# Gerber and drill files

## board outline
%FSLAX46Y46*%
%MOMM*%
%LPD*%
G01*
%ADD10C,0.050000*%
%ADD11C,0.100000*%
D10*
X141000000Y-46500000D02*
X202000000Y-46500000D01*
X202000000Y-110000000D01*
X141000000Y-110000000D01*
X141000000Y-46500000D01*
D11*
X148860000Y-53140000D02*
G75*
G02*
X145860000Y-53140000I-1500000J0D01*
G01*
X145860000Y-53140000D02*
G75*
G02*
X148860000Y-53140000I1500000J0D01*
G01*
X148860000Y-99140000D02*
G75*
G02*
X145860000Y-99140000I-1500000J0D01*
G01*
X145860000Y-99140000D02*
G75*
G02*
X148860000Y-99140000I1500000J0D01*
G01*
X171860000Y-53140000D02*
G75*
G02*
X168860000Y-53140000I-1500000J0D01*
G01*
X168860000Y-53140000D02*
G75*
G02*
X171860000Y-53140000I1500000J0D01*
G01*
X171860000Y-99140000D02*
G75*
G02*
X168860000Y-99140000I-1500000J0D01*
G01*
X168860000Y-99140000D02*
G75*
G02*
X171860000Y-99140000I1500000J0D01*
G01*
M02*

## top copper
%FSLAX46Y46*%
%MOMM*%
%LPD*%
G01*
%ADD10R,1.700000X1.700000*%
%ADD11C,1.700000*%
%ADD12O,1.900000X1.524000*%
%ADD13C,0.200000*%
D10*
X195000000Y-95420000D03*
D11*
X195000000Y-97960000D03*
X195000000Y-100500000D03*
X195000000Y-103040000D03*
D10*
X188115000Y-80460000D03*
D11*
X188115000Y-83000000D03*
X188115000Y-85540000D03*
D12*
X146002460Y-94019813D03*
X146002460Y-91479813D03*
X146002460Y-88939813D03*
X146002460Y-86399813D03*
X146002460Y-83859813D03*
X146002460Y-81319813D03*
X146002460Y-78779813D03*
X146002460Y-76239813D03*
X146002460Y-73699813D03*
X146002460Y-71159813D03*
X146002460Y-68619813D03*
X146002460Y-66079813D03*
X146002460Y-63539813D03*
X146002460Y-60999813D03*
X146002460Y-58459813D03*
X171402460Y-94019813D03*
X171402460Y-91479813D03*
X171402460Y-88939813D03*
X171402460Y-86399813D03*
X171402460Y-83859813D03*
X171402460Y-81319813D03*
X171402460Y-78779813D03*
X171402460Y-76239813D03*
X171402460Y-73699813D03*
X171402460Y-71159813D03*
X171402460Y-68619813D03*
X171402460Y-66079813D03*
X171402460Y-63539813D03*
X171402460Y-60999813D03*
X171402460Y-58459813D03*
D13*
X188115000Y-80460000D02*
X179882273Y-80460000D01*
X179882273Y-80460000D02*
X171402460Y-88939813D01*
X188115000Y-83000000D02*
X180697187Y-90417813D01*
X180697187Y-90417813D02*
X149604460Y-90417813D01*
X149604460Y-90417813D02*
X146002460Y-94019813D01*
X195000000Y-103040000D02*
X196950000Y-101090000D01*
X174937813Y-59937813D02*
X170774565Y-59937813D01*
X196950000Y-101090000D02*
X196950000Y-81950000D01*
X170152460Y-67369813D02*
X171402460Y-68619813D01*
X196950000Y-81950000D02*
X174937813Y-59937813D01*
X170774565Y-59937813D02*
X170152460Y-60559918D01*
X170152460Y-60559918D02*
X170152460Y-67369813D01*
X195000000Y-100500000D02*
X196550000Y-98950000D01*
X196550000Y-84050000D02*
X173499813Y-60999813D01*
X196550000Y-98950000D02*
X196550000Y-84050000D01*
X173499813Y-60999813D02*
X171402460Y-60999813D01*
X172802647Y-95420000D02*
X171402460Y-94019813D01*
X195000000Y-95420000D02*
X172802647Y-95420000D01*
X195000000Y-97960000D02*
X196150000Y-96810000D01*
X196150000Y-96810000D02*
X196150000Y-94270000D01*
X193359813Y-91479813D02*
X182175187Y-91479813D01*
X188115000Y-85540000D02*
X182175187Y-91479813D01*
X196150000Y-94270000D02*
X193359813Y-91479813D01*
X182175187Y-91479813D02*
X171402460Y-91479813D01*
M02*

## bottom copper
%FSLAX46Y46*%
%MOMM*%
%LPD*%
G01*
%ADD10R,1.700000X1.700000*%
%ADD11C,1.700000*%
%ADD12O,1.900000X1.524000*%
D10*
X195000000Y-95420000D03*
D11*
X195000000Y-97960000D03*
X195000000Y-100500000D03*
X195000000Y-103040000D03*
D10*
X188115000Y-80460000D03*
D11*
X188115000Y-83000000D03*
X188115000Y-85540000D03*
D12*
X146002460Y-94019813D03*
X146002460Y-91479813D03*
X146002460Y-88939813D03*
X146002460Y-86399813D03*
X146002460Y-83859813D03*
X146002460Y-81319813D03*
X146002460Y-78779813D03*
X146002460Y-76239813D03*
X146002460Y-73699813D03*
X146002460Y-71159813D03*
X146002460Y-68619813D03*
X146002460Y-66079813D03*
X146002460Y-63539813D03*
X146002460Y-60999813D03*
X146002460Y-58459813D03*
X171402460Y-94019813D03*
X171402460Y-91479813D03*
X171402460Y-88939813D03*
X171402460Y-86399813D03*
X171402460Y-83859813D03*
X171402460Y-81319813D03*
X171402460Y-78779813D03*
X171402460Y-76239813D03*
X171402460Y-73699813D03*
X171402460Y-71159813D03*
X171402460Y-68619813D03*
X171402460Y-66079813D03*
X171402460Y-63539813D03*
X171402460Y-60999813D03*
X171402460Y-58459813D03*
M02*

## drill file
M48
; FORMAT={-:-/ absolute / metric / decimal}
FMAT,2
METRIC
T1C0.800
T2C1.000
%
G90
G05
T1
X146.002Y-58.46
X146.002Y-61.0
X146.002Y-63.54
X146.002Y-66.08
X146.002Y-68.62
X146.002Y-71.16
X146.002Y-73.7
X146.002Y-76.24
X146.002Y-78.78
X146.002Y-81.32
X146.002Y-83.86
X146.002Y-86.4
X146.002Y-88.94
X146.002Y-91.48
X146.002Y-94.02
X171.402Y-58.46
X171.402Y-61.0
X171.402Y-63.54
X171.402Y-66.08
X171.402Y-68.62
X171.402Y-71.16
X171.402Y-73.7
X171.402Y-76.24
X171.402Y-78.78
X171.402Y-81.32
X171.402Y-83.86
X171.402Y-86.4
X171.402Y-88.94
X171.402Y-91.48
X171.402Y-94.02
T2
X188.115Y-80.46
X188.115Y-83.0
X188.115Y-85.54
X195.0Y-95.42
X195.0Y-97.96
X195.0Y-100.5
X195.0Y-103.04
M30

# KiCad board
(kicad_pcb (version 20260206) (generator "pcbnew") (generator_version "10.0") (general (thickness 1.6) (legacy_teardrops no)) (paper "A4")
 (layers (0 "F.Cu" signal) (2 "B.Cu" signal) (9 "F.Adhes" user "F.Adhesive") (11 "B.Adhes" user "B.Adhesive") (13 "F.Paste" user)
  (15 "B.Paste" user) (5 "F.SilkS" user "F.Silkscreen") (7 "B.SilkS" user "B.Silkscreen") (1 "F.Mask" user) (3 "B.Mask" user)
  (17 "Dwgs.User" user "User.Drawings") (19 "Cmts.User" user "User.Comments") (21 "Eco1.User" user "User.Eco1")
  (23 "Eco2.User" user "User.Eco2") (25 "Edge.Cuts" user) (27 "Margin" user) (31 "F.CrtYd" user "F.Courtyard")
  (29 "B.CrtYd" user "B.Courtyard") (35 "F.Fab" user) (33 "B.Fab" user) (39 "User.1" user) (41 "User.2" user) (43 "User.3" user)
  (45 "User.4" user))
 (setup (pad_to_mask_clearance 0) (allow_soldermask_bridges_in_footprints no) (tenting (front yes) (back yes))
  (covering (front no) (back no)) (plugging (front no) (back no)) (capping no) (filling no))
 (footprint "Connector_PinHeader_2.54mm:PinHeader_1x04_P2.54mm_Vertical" (layer "F.Cu") (at 195 95.42)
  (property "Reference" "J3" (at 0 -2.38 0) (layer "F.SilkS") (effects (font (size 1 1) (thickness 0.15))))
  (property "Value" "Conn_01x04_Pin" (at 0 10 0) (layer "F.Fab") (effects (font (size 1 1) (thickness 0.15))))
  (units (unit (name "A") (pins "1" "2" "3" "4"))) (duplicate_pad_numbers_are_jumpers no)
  (pad "1" thru_hole rect (at 0 0) (size 1.7 1.7) (drill 1) (layers "*.Cu" "*.Mask") (remove_unused_layers no) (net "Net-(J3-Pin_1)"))
  (pad "2" thru_hole circle (at 0 2.54) (size 1.7 1.7) (drill 1) (layers "*.Cu" "*.Mask") (remove_unused_layers no) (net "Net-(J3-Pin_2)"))
  (pad "3" thru_hole circle (at 0 5.08) (size 1.7 1.7) (drill 1) (layers "*.Cu" "*.Mask") (remove_unused_layers no) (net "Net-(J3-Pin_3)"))
  (pad "4" thru_hole circle (at 0 7.62) (size 1.7 1.7) (drill 1) (layers "*.Cu" "*.Mask") (remove_unused_layers no) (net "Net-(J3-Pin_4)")))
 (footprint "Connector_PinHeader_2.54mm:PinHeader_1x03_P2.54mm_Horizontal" (layer "F.Cu") (at 188.115 80.46)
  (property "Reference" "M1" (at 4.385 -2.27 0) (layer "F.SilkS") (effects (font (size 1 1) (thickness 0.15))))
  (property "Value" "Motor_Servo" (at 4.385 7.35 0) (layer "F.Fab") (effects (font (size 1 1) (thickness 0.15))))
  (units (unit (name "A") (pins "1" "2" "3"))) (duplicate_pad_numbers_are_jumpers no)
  (pad "1" thru_hole rect (at 0 0) (size 1.7 1.7) (drill 1) (layers "*.Cu" "*.Mask") (remove_unused_layers no) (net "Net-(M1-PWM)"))
  (pad "2" thru_hole circle (at 0 2.54) (size 1.7 1.7) (drill 1) (layers "*.Cu" "*.Mask") (remove_unused_layers no) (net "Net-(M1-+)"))
  (pad "3" thru_hole circle (at 0 5.08) (size 1.7 1.7) (drill 1) (layers "*.Cu" "*.Mask") (remove_unused_layers no) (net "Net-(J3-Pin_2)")))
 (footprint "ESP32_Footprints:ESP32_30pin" (layer "F.Cu") (at 157.93 77)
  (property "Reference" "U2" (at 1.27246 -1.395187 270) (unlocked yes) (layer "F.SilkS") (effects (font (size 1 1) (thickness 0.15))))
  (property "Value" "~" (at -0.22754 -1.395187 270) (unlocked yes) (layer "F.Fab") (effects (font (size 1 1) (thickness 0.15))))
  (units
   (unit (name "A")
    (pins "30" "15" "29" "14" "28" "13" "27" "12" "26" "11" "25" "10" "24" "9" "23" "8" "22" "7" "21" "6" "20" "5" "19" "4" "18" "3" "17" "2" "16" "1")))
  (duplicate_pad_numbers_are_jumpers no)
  (fp_circle (center -10.57 -23.86) (end -10.57 -22.36) (stroke (width 0.1) (type default)) (fill no) (layer "Edge.Cuts"))
  (fp_circle (center -10.57 22.14) (end -10.57 23.64) (stroke (width 0.1) (type default)) (fill no) (layer "Edge.Cuts"))
  (fp_circle (center 12.43 -23.86) (end 12.43 -22.36) (stroke (width 0.1) (type default)) (fill no) (layer "Edge.Cuts"))
  (fp_circle (center 12.43 22.14) (end 12.43 23.64) (stroke (width 0.1) (type default)) (fill no) (layer "Edge.Cuts"))
  (pad "1" thru_hole oval (at -11.92754 17.019813 270) (size 1.524 1.9) (drill 0.8) (layers "*.Cu" "*.Mask") (remove_unused_layers no)
   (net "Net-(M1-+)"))
  (pad "2" thru_hole oval (at -11.92754 14.479813 270) (size 1.524 1.9) (drill 0.8) (layers "*.Cu" "*.Mask") (remove_unused_layers no)
   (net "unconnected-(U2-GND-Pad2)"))
  (pad "3" thru_hole oval (at -11.92754 11.939813 270) (size 1.524 1.9) (drill 0.8) (layers "*.Cu" "*.Mask") (remove_unused_layers no)
   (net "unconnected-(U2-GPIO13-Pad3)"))
  (pad "4" thru_hole oval (at -11.92754 9.399813 270) (size 1.524 1.9) (drill 0.8) (layers "*.Cu" "*.Mask") (remove_unused_layers no)
   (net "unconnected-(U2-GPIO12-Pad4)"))
  (pad "5" thru_hole oval (at -11.92754 6.859813 270) (size 1.524 1.9) (drill 0.8) (layers "*.Cu" "*.Mask") (remove_unused_layers no)
   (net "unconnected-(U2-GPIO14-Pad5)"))
  (pad "6" thru_hole oval (at -11.92754 4.319813 270) (size 1.524 1.9) (drill 0.8) (layers "*.Cu" "*.Mask") (remove_unused_layers no)
   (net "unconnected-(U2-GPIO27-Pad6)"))
  (pad "7" thru_hole oval (at -11.92754 1.779813 270) (size 1.524 1.9) (drill 0.8) (layers "*.Cu" "*.Mask") (remove_unused_layers no)
   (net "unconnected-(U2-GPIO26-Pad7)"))
  (pad "8" thru_hole oval (at -11.92754 -0.760187 270) (size 1.524 1.9) (drill 0.8) (layers "*.Cu" "*.Mask") (remove_unused_layers no)
   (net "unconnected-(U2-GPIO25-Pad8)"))
  (pad "9" thru_hole oval (at -11.92754 -3.300187 270) (size 1.524 1.9) (drill 0.8) (layers "*.Cu" "*.Mask") (remove_unused_layers no)
   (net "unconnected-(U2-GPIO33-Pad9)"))
  (pad "10" thru_hole oval (at -11.92754 -5.840187 270) (size 1.524 1.9) (drill 0.8) (layers "*.Cu" "*.Mask") (remove_unused_layers no)
   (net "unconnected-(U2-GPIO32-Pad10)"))
  (pad "11" thru_hole oval (at -11.92754 -8.380187 270) (size 1.524 1.9) (drill 0.8) (layers "*.Cu" "*.Mask") (remove_unused_layers no)
   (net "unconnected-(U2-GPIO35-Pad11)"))
  (pad "12" thru_hole oval (at -11.92754 -10.920187 270) (size 1.524 1.9) (drill 0.8) (layers "*.Cu" "*.Mask") (remove_unused_layers no)
   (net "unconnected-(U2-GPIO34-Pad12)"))
  (pad "13" thru_hole oval (at -11.92754 -13.460187 270) (size 1.524 1.9) (drill 0.8) (layers "*.Cu" "*.Mask") (remove_unused_layers no)
   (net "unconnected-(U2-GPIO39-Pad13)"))
  (pad "14" thru_hole oval (at -11.92754 -16.000187 270) (size 1.524 1.9) (drill 0.8) (layers "*.Cu" "*.Mask") (remove_unused_layers no)
   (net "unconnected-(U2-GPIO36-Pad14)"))
  (pad "15" thru_hole oval (at -11.92754 -18.540187 270) (size 1.524 1.9) (drill 0.8) (layers "*.Cu" "*.Mask") (remove_unused_layers no)
   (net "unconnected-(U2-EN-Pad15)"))
  (pad "16" thru_hole oval (at 13.47246 17.019813 270) (size 1.524 1.9) (drill 0.8) (layers "*.Cu" "*.Mask") (remove_unused_layers no)
   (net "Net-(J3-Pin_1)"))
  (pad "17" thru_hole oval (at 13.47246 14.479813 270) (size 1.524 1.9) (drill 0.8) (layers "*.Cu" "*.Mask") (remove_unused_layers no)
   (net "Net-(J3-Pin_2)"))
  (pad "18" thru_hole oval (at 13.47246 11.939813 270) (size 1.524 1.9) (drill 0.8) (layers "*.Cu" "*.Mask") (remove_unused_layers no)
   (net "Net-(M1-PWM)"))
  (pad "19" thru_hole oval (at 13.47246 9.399813 270) (size 1.524 1.9) (drill 0.8) (layers "*.Cu" "*.Mask") (remove_unused_layers no)
   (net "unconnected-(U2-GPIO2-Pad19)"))
  (pad "20" thru_hole oval (at 13.47246 6.859813 270) (size 1.524 1.9) (drill 0.8) (layers "*.Cu" "*.Mask" "Dwgs.User")
   (remove_unused_layers no) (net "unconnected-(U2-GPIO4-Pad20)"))
  (pad "21" thru_hole oval (at 13.47246 4.319813 270) (size 1.524 1.9) (drill 0.8) (layers "*.Cu" "*.Mask") (remove_unused_layers no)
   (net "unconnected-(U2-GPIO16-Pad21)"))
  (pad "22" thru_hole oval (at 13.47246 1.779813 270) (size 1.524 1.9) (drill 0.8) (layers "*.Cu" "*.Mask") (remove_unused_layers no)
   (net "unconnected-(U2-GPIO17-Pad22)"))
  (pad "23" thru_hole oval (at 13.47246 -0.760187 270) (size 1.524 1.9) (drill 0.8) (layers "*.Cu" "*.Mask") (remove_unused_layers no)
   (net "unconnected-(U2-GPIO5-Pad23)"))
  (pad "24" thru_hole oval (at 13.47246 -3.300187 270) (size 1.524 1.9) (drill 0.8) (layers "*.Cu" "*.Mask") (remove_unused_layers no)
   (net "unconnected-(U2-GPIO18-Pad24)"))
  (pad "25" thru_hole oval (at 13.47246 -5.840187 270) (size 1.524 1.9) (drill 0.8) (layers "*.Cu" "*.Mask") (remove_unused_layers no)
   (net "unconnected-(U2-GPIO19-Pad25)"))
  (pad "26" thru_hole oval (at 13.47246 -8.380187 270) (size 1.524 1.9) (drill 0.8) (layers "*.Cu" "*.Mask") (remove_unused_layers no)
   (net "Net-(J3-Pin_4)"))
  (pad "27" thru_hole oval (at 13.47246 -10.920187 270) (size 1.524 1.9) (drill 0.8) (layers "*.Cu" "*.Mask") (remove_unused_layers no)
   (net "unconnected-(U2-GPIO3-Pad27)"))
  (pad "28" thru_hole oval (at 13.47246 -13.460187 270) (size 1.524 1.9) (drill 0.8) (layers "*.Cu" "*.Mask") (remove_unused_layers no)
   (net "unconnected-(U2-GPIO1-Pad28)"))
  (pad "29" thru_hole oval (at 13.47246 -16.000187 270) (size 1.524 1.9) (drill 0.8) (layers "*.Cu" "*.Mask") (remove_unused_layers no)
   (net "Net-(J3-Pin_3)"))
  (pad "30" thru_hole oval (at 13.47246 -18.540187 270) (size 1.524 1.9) (drill 0.8) (layers "*.Cu" "*.Mask") (remove_unused_layers no)
   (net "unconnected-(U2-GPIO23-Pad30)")))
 (gr_rect (start 141 46.5) (end 202 110) (stroke (width 0.05) (type default)) (fill no) (layer "Edge.Cuts"))
 (segment (start 188.115 80.46) (end 179.882273 80.46) (width 0.2) (layer "F.Cu") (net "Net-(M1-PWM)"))
 (segment (start 179.882273 80.46) (end 171.40246 88.939813) (width 0.2) (layer "F.Cu") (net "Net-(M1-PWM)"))
 (segment (start 188.115 83) (end 180.697187 90.417813) (width 0.2) (layer "F.Cu") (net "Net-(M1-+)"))
 (segment (start 180.697187 90.417813) (end 149.60446 90.417813) (width 0.2) (layer "F.Cu") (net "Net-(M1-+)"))
 (segment (start 149.60446 90.417813) (end 146.00246 94.019813) (width 0.2) (layer "F.Cu") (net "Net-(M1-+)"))
 (segment (start 195 103.04) (end 196.95 101.09) (width 0.2) (layer "F.Cu") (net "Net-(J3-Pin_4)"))
 (segment (start 174.937813 59.937813) (end 170.774565 59.937813) (width 0.2) (layer "F.Cu") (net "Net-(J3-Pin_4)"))
 (segment (start 196.95 101.09) (end 196.95 81.95) (width 0.2) (layer "F.Cu") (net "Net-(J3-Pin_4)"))
 (segment (start 170.15246 67.369813) (end 171.40246 68.619813) (width 0.2) (layer "F.Cu") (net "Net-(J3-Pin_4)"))
 (segment (start 196.95 81.95) (end 174.937813 59.937813) (width 0.2) (layer "F.Cu") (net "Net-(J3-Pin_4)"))
 (segment (start 170.774565 59.937813) (end 170.15246 60.559918) (width 0.2) (layer "F.Cu") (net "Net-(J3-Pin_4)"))
 (segment (start 170.15246 60.559918) (end 170.15246 67.369813) (width 0.2) (layer "F.Cu") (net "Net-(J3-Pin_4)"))
 (segment (start 195 100.5) (end 196.55 98.95) (width 0.2) (layer "F.Cu") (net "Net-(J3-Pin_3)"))
 (segment (start 196.55 84.05) (end 173.499813 60.999813) (width 0.2) (layer "F.Cu") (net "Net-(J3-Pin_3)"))
 (segment (start 196.55 98.95) (end 196.55 84.05) (width 0.2) (layer "F.Cu") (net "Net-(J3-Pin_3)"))
 (segment (start 173.499813 60.999813) (end 171.40246 60.999813) (width 0.2) (layer "F.Cu") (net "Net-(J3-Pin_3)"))
 (segment (start 172.802647 95.42) (end 171.40246 94.019813) (width 0.2) (layer "F.Cu") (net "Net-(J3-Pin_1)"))
 (segment (start 195 95.42) (end 172.802647 95.42) (width 0.2) (layer "F.Cu") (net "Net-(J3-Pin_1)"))
 (segment (start 195 97.96) (end 196.15 96.81) (width 0.2) (layer "F.Cu") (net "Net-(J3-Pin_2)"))
 (segment (start 196.15 96.81) (end 196.15 94.27) (width 0.2) (layer "F.Cu") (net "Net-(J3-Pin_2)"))
 (segment (start 193.359813 91.479813) (end 182.175187 91.479813) (width 0.2) (layer "F.Cu") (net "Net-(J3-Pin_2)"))
 (segment (start 188.115 85.54) (end 182.175187 91.479813) (width 0.2) (layer "F.Cu") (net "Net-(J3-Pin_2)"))
 (segment (start 196.15 94.27) (end 193.359813 91.479813) (width 0.2) (layer "F.Cu") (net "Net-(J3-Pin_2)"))
 (segment (start 182.175187 91.479813) (end 171.40246 91.479813) (width 0.2) (layer "F.Cu") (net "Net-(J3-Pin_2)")))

